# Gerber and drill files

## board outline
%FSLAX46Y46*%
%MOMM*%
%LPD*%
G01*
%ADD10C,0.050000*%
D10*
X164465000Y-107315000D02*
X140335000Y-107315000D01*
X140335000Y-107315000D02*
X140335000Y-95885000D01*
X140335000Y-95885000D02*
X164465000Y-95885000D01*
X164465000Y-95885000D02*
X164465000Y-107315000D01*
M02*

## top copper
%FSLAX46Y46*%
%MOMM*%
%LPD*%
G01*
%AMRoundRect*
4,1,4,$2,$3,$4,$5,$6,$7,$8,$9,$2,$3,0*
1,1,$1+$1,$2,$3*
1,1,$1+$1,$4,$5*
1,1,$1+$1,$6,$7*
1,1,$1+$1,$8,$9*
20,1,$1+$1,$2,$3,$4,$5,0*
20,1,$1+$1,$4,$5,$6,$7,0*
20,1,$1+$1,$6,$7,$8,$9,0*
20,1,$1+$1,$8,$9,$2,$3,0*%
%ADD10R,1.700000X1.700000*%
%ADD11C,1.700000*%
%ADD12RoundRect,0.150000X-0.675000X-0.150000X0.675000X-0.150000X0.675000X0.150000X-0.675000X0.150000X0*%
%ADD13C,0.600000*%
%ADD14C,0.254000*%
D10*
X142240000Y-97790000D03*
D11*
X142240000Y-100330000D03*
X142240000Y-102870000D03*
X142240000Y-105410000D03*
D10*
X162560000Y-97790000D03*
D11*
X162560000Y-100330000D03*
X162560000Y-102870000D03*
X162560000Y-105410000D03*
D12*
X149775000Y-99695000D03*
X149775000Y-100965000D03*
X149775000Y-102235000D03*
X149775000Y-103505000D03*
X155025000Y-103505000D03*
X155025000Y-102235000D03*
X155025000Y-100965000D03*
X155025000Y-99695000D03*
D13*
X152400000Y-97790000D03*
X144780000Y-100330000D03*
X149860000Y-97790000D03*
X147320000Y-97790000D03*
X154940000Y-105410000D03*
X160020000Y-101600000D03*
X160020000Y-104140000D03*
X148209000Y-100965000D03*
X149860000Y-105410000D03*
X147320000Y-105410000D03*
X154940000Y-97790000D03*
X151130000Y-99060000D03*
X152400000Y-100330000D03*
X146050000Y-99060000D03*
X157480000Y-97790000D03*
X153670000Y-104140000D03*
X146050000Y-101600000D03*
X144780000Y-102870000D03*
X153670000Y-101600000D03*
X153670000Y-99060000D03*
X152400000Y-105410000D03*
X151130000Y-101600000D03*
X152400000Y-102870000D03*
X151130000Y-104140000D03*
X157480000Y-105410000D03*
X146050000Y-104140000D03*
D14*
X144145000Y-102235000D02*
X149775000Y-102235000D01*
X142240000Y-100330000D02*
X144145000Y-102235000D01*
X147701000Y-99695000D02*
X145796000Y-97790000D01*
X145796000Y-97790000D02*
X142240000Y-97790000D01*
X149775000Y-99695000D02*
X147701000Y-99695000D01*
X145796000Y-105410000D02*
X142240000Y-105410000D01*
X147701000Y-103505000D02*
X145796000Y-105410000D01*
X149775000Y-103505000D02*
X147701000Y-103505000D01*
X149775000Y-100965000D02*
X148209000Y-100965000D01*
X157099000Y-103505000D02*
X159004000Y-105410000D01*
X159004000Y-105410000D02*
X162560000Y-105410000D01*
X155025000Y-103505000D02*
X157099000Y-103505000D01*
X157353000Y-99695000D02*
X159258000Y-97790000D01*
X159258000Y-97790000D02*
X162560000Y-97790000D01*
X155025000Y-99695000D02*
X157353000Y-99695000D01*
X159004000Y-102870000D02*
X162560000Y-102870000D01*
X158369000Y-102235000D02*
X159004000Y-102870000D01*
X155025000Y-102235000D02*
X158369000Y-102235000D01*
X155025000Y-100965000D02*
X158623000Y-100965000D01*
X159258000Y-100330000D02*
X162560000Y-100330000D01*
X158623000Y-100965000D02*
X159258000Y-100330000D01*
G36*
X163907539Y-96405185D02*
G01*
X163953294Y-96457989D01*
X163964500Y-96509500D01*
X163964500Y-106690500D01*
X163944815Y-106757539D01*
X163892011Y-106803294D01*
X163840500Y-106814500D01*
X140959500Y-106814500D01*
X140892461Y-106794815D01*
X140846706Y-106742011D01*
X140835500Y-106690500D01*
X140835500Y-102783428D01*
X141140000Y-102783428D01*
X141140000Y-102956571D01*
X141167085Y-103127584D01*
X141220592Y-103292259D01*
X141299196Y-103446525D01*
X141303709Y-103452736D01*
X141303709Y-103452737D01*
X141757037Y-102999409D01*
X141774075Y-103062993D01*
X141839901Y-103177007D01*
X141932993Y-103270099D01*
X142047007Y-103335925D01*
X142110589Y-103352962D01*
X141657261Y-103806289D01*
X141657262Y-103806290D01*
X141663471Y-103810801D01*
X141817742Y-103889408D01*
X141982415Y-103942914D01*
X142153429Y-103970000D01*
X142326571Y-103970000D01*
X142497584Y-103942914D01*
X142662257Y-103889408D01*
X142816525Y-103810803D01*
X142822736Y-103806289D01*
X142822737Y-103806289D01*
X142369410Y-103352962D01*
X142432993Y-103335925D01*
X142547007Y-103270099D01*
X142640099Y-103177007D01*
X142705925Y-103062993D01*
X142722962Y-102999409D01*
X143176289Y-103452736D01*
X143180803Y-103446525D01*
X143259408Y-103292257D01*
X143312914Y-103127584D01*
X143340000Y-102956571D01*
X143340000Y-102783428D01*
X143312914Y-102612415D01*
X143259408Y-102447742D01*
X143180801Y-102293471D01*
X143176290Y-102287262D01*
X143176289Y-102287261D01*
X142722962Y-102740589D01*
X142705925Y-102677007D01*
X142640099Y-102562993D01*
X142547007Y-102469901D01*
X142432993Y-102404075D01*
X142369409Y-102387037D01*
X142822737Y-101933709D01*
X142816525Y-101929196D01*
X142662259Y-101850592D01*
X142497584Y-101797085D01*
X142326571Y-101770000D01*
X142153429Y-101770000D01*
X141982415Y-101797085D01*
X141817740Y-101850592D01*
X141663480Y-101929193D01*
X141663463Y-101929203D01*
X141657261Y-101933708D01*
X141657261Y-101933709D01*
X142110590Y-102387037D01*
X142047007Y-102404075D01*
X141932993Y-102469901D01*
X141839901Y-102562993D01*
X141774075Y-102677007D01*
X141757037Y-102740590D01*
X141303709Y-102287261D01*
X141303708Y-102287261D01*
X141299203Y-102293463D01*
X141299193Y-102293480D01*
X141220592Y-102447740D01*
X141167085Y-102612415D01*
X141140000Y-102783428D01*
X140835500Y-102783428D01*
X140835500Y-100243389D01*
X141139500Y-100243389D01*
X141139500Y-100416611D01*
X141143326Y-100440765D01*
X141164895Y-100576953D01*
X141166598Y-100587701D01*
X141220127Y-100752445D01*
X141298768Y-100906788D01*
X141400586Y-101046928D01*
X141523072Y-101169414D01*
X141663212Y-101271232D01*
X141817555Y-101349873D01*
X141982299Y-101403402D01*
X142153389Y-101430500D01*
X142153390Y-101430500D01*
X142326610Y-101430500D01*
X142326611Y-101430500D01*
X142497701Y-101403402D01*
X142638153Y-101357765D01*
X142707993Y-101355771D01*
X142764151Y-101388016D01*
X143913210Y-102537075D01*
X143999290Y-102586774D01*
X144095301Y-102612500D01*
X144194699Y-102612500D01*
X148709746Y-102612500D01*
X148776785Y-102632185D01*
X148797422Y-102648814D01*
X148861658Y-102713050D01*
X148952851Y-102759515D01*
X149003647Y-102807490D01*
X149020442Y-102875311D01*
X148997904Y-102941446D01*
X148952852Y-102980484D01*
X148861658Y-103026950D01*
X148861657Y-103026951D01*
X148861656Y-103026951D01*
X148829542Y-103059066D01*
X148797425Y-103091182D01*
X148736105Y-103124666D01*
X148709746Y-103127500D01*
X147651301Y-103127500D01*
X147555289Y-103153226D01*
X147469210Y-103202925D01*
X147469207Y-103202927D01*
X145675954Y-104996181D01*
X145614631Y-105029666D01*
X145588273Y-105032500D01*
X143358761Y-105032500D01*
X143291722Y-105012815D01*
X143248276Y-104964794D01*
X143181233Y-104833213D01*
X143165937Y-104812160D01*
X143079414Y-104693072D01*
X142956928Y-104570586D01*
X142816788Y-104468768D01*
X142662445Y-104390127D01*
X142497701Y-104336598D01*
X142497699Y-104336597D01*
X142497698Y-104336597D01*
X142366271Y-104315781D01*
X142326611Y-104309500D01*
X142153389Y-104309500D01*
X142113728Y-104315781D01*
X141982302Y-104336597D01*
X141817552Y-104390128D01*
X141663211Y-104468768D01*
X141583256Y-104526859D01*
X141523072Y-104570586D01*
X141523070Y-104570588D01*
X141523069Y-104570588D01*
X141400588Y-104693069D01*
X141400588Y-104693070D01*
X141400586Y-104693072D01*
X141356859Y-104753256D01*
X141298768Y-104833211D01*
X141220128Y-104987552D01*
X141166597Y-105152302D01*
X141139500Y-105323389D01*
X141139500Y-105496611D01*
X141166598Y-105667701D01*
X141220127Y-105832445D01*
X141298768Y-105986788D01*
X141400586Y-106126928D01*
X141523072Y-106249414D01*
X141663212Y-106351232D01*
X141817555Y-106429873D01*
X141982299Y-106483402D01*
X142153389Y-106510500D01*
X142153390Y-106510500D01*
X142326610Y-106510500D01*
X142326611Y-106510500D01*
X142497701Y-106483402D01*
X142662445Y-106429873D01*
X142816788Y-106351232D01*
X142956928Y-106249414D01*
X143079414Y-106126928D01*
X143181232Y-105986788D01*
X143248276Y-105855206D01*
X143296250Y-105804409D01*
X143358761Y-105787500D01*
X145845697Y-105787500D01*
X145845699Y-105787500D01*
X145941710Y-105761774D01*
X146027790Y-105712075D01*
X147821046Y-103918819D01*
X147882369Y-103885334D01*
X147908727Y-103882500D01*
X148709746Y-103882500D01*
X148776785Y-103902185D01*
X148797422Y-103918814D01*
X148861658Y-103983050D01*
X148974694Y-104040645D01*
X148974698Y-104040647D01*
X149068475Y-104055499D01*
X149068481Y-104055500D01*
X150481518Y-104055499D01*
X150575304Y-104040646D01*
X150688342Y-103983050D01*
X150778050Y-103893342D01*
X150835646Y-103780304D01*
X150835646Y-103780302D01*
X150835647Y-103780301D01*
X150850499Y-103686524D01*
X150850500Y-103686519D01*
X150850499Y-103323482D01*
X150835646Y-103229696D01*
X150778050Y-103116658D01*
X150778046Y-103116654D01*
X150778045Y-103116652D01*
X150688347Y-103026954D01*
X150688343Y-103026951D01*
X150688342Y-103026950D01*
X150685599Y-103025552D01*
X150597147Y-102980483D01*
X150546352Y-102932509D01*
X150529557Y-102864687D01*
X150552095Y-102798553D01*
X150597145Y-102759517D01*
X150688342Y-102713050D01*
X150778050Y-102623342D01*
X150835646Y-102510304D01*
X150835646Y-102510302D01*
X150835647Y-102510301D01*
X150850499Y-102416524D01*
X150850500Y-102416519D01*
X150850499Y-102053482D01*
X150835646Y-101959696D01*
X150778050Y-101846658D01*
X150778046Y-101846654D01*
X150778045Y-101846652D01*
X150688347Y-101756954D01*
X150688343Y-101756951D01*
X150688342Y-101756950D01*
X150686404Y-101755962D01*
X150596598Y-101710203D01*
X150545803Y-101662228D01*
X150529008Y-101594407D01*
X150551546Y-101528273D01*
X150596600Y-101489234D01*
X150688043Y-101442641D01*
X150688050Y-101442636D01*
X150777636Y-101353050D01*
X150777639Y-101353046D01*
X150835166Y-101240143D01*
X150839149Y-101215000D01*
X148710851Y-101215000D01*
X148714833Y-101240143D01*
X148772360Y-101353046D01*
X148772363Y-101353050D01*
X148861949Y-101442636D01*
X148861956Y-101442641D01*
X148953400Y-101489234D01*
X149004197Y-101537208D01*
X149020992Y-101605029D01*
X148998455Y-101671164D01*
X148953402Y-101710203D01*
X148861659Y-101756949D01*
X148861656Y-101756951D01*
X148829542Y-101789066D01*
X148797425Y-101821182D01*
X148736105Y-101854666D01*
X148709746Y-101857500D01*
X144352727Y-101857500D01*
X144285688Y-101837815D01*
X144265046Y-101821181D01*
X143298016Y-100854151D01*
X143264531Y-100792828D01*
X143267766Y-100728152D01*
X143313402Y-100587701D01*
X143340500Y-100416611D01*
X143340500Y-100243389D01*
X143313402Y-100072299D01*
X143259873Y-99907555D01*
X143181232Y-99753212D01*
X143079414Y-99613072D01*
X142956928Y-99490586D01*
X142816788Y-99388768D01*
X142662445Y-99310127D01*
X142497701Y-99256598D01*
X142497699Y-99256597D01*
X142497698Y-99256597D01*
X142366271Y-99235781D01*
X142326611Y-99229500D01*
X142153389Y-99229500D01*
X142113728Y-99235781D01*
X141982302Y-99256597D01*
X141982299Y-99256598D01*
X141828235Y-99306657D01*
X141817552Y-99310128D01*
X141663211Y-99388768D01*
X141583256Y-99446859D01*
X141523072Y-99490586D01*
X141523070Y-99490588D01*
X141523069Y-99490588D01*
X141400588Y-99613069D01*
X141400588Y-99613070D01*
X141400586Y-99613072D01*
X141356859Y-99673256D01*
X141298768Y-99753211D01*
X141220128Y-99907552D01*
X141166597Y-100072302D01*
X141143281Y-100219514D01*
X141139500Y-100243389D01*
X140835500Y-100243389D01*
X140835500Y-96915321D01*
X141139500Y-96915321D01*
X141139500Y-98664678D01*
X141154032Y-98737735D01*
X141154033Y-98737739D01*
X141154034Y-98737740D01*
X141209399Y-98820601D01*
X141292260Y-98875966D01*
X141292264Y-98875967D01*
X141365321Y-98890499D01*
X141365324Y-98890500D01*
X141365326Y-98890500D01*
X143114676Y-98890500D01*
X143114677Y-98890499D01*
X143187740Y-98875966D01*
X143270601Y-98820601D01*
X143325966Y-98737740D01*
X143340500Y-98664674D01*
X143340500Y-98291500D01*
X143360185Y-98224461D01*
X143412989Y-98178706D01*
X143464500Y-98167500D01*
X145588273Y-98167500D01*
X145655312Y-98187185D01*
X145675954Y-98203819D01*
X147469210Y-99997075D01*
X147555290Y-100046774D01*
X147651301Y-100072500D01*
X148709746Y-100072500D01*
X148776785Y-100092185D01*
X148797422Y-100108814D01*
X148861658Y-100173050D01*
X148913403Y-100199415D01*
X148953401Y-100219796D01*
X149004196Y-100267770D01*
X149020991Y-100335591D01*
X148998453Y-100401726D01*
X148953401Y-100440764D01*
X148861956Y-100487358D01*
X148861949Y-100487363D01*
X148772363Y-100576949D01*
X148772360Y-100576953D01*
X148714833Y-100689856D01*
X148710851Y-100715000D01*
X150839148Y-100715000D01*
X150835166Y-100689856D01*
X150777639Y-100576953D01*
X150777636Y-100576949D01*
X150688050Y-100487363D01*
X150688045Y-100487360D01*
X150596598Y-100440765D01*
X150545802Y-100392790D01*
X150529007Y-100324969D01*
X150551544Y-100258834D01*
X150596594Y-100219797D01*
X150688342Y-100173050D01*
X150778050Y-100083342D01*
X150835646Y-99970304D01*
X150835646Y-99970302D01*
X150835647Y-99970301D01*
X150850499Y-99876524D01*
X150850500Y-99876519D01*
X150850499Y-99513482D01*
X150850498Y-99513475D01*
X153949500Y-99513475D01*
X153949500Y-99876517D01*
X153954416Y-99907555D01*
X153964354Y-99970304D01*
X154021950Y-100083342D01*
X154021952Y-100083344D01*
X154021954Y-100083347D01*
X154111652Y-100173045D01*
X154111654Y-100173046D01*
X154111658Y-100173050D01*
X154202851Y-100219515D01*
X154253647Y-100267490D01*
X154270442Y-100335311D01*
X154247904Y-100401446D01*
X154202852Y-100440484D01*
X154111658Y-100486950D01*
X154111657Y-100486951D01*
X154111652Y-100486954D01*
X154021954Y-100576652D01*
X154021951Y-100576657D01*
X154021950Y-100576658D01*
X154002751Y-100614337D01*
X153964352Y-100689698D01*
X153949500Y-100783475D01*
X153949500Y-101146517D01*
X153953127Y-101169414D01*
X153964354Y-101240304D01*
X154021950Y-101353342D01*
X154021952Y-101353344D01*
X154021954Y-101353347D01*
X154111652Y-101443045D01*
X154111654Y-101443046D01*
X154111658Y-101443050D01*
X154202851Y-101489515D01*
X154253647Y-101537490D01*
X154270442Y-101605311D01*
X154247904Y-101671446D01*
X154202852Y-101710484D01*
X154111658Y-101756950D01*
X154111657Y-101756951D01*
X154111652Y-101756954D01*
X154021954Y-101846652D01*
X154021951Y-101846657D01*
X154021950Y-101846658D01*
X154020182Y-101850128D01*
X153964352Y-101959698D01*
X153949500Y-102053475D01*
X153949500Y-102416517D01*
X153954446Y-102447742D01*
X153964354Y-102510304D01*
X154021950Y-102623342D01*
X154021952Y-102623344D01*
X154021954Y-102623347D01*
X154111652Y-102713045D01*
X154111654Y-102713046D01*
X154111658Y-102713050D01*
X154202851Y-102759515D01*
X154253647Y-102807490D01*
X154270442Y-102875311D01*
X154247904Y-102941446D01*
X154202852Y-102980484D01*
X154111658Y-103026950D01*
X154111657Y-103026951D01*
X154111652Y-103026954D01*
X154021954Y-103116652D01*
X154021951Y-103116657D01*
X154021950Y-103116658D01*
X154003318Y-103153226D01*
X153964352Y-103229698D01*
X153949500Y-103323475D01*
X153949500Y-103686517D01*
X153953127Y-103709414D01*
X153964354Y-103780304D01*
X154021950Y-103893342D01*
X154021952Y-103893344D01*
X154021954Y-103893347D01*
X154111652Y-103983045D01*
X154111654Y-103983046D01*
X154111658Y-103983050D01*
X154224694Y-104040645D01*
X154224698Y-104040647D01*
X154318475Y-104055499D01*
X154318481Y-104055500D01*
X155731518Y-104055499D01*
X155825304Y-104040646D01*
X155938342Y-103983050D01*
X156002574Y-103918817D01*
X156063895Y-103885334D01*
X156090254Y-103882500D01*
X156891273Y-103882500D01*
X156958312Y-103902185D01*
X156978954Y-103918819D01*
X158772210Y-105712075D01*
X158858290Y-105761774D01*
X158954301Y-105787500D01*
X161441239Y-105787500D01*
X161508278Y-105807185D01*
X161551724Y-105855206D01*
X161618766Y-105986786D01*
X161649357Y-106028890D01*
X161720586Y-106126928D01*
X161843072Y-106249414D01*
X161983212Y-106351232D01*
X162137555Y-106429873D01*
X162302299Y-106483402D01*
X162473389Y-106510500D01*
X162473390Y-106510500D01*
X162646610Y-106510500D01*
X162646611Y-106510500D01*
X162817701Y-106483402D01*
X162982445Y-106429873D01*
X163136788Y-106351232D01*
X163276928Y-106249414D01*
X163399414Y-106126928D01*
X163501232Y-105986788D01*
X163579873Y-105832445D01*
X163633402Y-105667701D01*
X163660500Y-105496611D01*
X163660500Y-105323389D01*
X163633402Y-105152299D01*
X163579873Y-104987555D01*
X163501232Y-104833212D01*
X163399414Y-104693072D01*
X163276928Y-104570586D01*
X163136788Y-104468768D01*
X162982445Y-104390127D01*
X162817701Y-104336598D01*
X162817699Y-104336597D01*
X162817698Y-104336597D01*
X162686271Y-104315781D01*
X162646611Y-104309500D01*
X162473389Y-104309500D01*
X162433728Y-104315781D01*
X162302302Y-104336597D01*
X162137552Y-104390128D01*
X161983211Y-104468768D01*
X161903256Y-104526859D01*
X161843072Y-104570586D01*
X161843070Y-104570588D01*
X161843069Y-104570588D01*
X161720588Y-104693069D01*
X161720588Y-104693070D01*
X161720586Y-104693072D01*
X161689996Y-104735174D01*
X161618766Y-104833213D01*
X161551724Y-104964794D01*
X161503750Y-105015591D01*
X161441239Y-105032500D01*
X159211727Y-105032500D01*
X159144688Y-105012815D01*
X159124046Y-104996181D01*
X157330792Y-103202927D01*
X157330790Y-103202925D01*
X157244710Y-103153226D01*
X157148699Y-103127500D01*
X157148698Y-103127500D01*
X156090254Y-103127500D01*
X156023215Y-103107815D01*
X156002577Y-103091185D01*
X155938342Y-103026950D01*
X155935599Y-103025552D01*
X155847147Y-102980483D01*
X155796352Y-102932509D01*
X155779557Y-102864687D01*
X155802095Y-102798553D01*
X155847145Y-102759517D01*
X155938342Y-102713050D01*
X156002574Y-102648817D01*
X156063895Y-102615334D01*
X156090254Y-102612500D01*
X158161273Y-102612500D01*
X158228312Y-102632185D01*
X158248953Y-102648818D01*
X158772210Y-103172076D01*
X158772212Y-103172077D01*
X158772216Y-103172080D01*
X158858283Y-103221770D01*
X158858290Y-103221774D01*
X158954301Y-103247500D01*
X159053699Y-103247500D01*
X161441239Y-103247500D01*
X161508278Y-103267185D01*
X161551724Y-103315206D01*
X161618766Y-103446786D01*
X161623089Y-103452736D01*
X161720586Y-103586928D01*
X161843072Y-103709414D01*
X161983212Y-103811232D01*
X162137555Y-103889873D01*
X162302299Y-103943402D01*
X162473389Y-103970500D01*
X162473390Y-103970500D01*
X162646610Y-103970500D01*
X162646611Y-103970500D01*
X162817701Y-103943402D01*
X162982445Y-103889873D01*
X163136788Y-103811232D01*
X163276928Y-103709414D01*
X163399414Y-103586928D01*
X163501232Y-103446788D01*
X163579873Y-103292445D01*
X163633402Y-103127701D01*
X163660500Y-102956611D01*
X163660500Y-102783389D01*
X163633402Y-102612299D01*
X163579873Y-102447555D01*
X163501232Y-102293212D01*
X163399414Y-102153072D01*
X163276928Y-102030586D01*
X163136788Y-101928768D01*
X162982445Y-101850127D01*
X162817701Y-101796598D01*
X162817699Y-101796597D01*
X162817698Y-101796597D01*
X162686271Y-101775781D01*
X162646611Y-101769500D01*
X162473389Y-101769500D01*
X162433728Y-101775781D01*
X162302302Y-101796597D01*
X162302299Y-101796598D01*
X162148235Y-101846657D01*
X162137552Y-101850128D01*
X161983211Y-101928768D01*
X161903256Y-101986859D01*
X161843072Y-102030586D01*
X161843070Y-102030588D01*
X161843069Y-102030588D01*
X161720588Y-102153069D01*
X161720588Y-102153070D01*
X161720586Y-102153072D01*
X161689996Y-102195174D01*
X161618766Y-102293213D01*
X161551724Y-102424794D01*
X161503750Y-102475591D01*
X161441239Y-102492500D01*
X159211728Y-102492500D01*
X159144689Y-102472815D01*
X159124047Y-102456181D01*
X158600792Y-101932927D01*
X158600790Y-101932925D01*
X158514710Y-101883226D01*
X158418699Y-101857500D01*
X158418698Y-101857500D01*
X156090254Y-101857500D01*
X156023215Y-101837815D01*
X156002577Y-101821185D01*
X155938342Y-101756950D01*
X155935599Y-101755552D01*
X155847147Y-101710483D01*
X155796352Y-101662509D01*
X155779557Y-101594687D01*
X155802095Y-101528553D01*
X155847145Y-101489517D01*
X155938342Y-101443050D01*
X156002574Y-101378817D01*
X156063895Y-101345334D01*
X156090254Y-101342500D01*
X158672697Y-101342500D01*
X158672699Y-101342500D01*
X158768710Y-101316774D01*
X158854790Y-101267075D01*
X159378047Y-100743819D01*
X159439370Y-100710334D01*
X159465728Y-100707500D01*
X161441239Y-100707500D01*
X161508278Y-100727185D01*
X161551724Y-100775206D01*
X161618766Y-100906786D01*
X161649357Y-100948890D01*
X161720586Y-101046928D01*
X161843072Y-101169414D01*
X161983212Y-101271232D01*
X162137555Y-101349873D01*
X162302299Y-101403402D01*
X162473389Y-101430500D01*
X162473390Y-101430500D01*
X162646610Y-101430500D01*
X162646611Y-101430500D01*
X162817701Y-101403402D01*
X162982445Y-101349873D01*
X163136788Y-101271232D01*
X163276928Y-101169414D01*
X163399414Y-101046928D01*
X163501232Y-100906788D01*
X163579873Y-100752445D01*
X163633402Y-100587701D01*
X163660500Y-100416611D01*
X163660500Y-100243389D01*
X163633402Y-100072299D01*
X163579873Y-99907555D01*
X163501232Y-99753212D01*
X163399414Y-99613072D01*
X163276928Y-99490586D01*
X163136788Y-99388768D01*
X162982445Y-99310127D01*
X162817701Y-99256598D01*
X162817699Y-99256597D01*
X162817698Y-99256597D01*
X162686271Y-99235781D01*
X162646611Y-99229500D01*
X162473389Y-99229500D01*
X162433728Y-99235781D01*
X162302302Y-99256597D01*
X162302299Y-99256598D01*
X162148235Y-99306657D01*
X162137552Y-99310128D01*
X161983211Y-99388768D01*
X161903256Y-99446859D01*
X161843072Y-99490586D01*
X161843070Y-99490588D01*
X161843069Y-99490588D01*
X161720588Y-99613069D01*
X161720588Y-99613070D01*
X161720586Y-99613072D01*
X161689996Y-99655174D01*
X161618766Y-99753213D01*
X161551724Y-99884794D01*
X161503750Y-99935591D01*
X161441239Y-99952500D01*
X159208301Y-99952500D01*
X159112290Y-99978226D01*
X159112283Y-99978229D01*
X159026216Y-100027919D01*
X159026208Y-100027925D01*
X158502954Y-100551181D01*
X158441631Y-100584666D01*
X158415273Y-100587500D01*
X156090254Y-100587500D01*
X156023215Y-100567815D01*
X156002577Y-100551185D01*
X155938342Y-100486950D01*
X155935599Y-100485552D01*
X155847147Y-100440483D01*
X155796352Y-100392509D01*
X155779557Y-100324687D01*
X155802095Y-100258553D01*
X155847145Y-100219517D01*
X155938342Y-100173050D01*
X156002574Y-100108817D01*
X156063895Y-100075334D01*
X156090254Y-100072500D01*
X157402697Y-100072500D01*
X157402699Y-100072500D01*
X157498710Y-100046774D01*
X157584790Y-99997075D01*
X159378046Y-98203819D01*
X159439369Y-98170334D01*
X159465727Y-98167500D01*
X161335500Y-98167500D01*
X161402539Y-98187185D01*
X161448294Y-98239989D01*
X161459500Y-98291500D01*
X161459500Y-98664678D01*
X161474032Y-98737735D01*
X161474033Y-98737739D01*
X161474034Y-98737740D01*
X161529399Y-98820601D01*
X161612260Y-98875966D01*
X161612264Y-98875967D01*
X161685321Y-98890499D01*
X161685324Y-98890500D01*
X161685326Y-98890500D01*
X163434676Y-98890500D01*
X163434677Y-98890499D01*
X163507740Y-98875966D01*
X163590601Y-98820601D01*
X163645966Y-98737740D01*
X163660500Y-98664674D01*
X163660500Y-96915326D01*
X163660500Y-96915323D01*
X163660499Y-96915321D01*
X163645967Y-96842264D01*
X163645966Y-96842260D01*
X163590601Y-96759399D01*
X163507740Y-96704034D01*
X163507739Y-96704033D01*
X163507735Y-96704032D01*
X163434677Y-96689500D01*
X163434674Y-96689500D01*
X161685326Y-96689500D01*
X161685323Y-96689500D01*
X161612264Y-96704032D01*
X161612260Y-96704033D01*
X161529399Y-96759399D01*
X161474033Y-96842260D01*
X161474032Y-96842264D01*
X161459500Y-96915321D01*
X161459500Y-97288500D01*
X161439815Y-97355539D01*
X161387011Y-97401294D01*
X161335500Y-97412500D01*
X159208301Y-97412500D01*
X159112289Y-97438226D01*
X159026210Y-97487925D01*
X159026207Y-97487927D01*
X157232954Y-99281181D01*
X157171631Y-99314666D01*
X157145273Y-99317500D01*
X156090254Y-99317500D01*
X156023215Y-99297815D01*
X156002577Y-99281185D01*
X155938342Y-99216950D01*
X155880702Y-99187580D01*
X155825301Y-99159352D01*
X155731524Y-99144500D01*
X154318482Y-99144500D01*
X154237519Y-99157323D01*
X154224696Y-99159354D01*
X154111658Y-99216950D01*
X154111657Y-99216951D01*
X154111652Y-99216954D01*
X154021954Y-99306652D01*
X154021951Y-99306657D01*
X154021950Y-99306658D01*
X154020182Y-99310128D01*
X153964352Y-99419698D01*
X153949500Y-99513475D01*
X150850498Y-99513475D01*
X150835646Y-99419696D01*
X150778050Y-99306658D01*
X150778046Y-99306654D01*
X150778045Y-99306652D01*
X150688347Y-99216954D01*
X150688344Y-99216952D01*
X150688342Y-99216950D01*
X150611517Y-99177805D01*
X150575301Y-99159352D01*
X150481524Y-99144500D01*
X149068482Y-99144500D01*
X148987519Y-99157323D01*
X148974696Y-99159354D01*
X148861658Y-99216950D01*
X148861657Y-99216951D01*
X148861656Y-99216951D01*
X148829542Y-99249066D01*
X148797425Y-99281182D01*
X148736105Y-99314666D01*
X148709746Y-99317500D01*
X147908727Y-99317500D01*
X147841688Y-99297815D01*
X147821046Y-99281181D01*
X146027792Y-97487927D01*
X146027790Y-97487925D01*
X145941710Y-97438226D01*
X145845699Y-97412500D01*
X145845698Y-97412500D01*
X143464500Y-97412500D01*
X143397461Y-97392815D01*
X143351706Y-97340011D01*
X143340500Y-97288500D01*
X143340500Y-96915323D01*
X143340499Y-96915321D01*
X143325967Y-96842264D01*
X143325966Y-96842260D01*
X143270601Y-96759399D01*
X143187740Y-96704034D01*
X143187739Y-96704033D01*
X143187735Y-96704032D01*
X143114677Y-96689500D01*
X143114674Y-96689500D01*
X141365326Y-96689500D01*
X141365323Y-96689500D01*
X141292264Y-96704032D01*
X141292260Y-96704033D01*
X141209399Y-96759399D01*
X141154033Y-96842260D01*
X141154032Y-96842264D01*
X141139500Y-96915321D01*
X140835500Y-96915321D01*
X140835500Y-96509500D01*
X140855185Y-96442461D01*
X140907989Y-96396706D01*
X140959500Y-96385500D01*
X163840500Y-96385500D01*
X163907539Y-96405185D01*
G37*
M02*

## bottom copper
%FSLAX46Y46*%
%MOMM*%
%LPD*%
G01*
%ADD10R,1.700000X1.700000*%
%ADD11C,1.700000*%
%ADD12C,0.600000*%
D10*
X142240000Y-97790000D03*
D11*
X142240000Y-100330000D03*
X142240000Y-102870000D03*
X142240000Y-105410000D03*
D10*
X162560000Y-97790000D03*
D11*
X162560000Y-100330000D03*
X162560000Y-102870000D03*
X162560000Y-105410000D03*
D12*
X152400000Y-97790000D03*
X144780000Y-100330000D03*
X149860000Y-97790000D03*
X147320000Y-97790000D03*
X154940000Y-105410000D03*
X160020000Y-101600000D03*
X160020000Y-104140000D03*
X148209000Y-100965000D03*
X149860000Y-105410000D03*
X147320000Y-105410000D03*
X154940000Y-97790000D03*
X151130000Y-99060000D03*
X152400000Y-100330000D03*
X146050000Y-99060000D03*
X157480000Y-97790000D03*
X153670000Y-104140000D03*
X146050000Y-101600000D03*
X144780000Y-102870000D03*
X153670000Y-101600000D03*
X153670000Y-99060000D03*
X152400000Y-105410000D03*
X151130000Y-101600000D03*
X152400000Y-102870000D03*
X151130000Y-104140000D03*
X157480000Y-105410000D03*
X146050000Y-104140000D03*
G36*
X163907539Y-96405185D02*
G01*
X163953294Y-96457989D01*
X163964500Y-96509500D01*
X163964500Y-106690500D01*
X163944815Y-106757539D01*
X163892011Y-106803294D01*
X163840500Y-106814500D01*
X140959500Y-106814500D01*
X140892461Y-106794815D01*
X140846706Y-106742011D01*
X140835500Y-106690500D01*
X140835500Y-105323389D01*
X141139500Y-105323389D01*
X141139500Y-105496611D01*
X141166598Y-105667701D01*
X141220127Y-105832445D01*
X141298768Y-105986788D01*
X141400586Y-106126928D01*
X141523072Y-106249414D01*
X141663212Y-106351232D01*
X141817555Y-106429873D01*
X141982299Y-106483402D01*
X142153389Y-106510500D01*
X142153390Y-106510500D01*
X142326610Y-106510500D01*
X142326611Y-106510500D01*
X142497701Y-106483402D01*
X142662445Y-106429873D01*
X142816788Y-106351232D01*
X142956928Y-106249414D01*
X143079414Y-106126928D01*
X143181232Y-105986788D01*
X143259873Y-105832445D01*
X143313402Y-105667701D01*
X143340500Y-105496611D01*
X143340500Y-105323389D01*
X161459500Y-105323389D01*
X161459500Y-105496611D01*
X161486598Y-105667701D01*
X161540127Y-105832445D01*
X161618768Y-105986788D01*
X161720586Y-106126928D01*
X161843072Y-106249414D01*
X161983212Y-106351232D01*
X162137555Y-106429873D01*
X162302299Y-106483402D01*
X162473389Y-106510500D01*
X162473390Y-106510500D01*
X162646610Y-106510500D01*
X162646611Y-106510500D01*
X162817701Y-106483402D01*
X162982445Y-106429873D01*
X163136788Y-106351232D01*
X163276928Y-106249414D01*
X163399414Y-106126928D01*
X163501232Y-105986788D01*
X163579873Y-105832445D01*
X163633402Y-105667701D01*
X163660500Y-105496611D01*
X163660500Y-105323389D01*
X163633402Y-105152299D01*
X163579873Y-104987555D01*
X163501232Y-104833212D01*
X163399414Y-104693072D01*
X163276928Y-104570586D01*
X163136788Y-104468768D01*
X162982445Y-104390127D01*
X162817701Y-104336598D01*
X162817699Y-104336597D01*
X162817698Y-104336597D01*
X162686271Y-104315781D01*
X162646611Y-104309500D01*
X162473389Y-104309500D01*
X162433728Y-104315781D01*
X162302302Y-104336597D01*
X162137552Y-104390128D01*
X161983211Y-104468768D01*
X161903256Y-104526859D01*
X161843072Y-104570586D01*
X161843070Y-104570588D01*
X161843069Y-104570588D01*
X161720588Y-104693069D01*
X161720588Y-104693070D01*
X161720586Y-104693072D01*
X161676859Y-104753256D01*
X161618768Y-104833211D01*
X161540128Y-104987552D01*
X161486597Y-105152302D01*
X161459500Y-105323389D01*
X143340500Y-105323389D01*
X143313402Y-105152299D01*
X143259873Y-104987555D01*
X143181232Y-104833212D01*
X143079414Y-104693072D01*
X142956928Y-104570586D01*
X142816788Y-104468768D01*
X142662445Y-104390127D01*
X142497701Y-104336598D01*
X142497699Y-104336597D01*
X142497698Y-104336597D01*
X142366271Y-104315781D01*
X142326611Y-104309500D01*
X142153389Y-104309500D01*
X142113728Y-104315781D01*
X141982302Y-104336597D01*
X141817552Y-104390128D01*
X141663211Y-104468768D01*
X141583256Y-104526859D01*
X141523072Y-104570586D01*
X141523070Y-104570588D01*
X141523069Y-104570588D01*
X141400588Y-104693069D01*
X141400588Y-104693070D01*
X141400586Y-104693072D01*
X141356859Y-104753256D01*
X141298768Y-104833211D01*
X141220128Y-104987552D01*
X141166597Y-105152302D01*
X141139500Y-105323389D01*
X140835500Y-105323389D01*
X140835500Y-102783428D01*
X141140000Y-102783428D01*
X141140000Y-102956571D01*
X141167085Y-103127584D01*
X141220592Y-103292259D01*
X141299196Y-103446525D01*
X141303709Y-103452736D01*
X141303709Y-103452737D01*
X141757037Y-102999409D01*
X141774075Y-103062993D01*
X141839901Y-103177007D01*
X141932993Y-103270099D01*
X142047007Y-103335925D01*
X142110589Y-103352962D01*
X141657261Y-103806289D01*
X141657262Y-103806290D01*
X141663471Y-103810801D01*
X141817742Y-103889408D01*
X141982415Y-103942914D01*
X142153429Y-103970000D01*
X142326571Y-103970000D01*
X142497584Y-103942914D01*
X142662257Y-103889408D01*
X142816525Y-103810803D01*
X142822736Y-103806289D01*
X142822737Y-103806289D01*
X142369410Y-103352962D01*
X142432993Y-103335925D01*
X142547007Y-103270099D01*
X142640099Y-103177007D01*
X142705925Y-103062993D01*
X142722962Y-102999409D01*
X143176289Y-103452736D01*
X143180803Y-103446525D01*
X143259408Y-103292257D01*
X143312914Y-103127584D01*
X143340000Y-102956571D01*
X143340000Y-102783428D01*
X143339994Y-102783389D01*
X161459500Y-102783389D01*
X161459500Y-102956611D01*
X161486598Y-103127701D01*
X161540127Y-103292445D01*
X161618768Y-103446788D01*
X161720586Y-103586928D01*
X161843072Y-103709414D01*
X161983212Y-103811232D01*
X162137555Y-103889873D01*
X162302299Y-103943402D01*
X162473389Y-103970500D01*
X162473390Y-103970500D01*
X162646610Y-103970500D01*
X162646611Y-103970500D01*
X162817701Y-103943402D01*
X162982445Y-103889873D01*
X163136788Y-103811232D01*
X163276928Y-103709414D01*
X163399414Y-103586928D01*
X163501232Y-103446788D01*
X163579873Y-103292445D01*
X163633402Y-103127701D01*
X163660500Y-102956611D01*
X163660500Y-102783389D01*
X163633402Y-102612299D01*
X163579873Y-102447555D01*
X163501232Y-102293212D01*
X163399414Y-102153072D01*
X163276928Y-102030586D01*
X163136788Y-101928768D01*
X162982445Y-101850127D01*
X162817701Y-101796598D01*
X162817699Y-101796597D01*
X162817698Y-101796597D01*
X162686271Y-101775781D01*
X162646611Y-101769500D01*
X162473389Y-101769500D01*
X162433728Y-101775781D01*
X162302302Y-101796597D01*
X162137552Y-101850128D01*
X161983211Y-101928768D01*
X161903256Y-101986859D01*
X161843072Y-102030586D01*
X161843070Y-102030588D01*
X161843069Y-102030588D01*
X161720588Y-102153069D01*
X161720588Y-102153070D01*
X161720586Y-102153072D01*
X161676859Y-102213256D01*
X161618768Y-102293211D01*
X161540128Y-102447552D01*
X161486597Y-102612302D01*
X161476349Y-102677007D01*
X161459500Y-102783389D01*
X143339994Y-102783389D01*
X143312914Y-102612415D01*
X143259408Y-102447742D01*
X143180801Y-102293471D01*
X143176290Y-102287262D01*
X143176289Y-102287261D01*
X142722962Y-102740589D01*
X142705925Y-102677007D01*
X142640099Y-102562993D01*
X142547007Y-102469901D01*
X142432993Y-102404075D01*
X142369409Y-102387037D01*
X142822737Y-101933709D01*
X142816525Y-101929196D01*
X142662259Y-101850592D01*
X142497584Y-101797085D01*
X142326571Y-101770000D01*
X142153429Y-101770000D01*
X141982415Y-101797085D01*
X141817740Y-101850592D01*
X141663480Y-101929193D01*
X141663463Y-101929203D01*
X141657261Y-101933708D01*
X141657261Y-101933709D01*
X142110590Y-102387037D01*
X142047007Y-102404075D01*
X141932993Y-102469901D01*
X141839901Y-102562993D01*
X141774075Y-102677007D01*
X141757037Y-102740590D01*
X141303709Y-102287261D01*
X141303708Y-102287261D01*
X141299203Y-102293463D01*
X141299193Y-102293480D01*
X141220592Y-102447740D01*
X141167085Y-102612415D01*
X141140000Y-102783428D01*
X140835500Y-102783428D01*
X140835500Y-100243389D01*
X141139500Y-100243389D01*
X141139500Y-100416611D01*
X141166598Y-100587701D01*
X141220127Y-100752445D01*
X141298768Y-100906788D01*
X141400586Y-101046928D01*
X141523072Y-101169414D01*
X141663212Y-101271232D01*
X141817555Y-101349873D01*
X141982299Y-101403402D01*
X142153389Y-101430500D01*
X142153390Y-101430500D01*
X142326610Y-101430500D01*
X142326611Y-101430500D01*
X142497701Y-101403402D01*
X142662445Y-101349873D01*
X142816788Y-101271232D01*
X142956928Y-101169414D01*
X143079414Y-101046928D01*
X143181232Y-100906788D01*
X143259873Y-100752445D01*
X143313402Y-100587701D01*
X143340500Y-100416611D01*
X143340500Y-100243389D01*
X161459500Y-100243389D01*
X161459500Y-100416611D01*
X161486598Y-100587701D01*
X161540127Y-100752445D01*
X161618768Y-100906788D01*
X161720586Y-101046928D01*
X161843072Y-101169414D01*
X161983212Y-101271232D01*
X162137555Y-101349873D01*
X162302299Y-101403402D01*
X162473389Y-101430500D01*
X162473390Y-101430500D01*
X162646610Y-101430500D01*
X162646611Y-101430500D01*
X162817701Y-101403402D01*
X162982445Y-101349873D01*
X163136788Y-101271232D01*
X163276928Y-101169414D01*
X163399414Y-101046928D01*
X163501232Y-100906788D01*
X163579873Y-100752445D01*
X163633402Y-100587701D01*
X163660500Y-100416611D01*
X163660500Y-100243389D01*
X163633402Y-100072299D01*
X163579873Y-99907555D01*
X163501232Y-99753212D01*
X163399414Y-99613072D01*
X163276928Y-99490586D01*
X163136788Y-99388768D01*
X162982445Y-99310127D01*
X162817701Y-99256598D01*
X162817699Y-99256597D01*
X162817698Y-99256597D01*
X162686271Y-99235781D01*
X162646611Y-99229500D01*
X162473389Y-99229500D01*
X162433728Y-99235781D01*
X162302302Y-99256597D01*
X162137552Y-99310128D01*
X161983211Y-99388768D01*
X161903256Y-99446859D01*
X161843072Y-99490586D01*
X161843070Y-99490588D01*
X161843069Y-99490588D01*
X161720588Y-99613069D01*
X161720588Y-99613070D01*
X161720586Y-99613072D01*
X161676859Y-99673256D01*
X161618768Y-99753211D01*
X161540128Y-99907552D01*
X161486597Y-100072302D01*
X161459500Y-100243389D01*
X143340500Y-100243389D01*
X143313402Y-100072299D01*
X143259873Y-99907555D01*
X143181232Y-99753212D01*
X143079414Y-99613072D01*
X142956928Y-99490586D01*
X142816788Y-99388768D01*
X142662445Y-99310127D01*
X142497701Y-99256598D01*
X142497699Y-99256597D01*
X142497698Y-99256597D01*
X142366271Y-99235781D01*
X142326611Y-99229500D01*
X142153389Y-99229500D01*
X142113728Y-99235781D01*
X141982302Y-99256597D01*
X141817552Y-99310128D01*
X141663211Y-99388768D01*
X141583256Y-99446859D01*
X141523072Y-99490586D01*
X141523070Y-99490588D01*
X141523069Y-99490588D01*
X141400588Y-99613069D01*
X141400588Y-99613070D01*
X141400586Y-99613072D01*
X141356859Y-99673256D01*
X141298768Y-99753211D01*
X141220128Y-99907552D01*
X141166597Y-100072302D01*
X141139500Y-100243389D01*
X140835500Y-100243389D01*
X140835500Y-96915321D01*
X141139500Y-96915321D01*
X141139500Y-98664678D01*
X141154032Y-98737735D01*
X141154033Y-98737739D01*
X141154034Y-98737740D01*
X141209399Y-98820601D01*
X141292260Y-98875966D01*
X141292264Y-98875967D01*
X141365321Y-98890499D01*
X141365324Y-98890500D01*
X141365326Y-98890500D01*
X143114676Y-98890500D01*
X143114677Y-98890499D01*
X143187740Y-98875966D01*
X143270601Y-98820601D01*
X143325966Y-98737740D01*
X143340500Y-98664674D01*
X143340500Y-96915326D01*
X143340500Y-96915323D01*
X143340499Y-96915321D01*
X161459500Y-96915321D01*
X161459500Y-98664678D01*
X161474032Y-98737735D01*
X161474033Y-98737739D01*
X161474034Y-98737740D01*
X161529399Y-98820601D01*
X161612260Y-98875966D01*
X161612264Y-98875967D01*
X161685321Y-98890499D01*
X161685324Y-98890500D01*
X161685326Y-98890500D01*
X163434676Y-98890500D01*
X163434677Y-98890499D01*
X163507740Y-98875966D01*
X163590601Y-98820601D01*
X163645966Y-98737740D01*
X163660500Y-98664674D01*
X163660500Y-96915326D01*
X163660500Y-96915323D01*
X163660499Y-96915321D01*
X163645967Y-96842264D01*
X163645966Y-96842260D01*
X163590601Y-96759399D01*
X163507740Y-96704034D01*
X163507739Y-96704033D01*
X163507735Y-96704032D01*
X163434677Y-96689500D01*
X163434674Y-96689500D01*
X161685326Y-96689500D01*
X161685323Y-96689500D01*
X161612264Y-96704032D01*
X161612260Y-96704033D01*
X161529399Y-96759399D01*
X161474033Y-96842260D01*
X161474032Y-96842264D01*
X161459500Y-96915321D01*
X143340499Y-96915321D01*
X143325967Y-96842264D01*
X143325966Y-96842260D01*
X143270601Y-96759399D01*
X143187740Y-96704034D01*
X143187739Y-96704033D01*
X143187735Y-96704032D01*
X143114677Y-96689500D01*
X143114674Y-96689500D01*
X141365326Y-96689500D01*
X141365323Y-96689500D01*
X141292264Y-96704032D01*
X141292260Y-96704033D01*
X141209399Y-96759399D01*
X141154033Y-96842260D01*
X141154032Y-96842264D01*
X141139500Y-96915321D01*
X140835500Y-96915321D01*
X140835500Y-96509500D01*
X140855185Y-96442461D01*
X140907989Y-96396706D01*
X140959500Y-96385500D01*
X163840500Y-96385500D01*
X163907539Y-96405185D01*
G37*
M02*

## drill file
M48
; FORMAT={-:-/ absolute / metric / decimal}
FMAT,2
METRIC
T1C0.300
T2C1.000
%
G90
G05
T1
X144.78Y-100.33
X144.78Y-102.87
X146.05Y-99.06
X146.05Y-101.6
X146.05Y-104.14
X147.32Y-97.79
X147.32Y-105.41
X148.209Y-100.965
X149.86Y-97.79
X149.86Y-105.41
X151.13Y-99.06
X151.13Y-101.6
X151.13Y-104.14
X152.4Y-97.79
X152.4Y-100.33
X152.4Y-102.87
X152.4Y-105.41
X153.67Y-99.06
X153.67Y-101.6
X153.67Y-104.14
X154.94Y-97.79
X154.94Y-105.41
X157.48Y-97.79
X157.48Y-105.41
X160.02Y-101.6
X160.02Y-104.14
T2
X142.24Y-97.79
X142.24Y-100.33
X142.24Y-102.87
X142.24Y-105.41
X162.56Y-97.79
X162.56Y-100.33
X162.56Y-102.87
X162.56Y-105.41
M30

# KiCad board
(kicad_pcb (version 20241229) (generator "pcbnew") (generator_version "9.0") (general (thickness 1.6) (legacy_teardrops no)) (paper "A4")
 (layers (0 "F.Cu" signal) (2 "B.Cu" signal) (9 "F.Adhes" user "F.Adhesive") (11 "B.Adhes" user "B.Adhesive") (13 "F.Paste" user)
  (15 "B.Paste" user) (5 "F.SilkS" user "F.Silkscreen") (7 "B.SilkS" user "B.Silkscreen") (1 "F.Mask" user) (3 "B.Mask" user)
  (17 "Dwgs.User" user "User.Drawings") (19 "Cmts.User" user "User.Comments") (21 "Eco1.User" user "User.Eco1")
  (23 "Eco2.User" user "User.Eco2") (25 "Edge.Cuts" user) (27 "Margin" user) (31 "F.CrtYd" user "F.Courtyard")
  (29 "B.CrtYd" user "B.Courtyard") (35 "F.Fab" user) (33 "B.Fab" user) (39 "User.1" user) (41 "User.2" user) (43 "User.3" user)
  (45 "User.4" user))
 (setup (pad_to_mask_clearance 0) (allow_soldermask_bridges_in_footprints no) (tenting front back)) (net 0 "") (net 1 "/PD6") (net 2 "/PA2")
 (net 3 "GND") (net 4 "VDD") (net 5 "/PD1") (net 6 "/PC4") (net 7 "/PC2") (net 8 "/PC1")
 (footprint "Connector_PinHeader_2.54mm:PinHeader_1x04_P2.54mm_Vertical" (layer "F.Cu") (at 142.24 97.79)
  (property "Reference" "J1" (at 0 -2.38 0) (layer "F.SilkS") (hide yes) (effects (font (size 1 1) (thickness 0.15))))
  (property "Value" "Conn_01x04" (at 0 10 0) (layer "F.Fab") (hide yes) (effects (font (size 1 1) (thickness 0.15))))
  (pad "1" thru_hole rect (at 0 0) (size 1.7 1.7) (drill 1) (layers "*.Cu" "*.Mask") (remove_unused_layers no) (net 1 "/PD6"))
  (pad "2" thru_hole circle (at 0 2.54) (size 1.7 1.7) (drill 1) (layers "*.Cu" "*.Mask") (remove_unused_layers no) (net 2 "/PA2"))
  (pad "3" thru_hole circle (at 0 5.08) (size 1.7 1.7) (drill 1) (layers "*.Cu" "*.Mask") (remove_unused_layers no) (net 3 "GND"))
  (pad "4" thru_hole circle (at 0 7.62) (size 1.7 1.7) (drill 1) (layers "*.Cu" "*.Mask") (remove_unused_layers no) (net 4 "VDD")))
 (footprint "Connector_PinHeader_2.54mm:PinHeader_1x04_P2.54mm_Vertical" (layer "F.Cu") (at 162.56 97.79)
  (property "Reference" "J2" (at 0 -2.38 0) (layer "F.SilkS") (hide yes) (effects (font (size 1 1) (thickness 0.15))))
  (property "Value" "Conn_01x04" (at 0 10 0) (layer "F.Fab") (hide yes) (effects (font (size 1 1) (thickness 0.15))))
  (pad "1" thru_hole rect (at 0 0) (size 1.7 1.7) (drill 1) (layers "*.Cu" "*.Mask") (remove_unused_layers no) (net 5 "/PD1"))
  (pad "2" thru_hole circle (at 0 2.54) (size 1.7 1.7) (drill 1) (layers "*.Cu" "*.Mask") (remove_unused_layers no) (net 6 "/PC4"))
  (pad "3" thru_hole circle (at 0 5.08) (size 1.7 1.7) (drill 1) (layers "*.Cu" "*.Mask") (remove_unused_layers no) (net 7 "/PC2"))
  (pad "4" thru_hole circle (at 0 7.62) (size 1.7 1.7) (drill 1) (layers "*.Cu" "*.Mask") (remove_unused_layers no) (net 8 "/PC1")))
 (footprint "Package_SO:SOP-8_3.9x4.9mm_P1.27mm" (layer "F.Cu") (at 152.4 101.6)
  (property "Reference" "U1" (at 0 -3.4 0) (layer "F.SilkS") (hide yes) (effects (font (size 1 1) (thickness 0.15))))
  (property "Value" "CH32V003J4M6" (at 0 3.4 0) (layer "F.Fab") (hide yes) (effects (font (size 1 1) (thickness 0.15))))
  (pad "1" smd roundrect (at -2.625 -1.905) (size 1.65 0.6) (layers "F.Cu" "F.Mask" "F.Paste") (roundrect_rratio 0.25) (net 1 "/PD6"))
  (pad "2" smd roundrect (at -2.625 -0.635) (size 1.65 0.6) (layers "F.Cu" "F.Mask" "F.Paste") (roundrect_rratio 0.25) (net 3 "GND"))
  (pad "3" smd roundrect (at -2.625 0.635) (size 1.65 0.6) (layers "F.Cu" "F.Mask" "F.Paste") (roundrect_rratio 0.25) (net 2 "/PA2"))
  (pad "4" smd roundrect (at -2.625 1.905) (size 1.65 0.6) (layers "F.Cu" "F.Mask" "F.Paste") (roundrect_rratio 0.25) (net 4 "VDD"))
  (pad "5" smd roundrect (at 2.625 1.905) (size 1.65 0.6) (layers "F.Cu" "F.Mask" "F.Paste") (roundrect_rratio 0.25) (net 8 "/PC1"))
  (pad "6" smd roundrect (at 2.625 0.635) (size 1.65 0.6) (layers "F.Cu" "F.Mask" "F.Paste") (roundrect_rratio 0.25) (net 7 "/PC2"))
  (pad "7" smd roundrect (at 2.625 -0.635) (size 1.65 0.6) (layers "F.Cu" "F.Mask" "F.Paste") (roundrect_rratio 0.25) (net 6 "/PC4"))
  (pad "8" smd roundrect (at 2.625 -1.905) (size 1.65 0.6) (layers "F.Cu" "F.Mask" "F.Paste") (roundrect_rratio 0.25) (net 5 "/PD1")))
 (gr_line (start 164.465 107.315) (end 140.335 107.315) (stroke (width 0.05) (type default)) (layer "Edge.Cuts"))
 (gr_line (start 140.335 107.315) (end 140.335 95.885) (stroke (width 0.05) (type default)) (layer "Edge.Cuts"))
 (gr_line (start 140.335 95.885) (end 164.465 95.885) (stroke (width 0.05) (type default)) (layer "Edge.Cuts"))
 (gr_line (start 164.465 95.885) (end 164.465 107.315) (stroke (width 0.05) (type default)) (layer "Edge.Cuts"))
 (segment (start 144.145 102.235) (end 149.775 102.235) (width 0.254) (layer "F.Cu") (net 2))
 (segment (start 142.24 100.33) (end 144.145 102.235) (width 0.254) (layer "F.Cu") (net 2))
 (segment (start 147.701 99.695) (end 145.796 97.79) (width 0.254) (layer "F.Cu") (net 1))
 (segment (start 145.796 97.79) (end 142.24 97.79) (width 0.254) (layer "F.Cu") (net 1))
 (segment (start 149.775 99.695) (end 147.701 99.695) (width 0.254) (layer "F.Cu") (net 1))
 (segment (start 145.796 105.41) (end 142.24 105.41) (width 0.254) (layer "F.Cu") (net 4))
 (segment (start 147.701 103.505) (end 145.796 105.41) (width 0.254) (layer "F.Cu") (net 4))
 (segment (start 149.775 103.505) (end 147.701 103.505) (width 0.254) (layer "F.Cu") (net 4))
 (segment (start 149.775 100.965) (end 148.209 100.965) (width 0.254) (layer "F.Cu") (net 3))
 (via (at 152.4 97.79) (size 0.6) (drill 0.3) (layers "F.Cu" "B.Cu") (free yes) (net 3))
 (via (at 144.78 100.33) (size 0.6) (drill 0.3) (layers "F.Cu" "B.Cu") (free yes) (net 3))
 (via (at 149.86 97.79) (size 0.6) (drill 0.3) (layers "F.Cu" "B.Cu") (free yes) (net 3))
 (via (at 147.32 97.79) (size 0.6) (drill 0.3) (layers "F.Cu" "B.Cu") (free yes) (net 3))
 (via (at 154.94 105.41) (size 0.6) (drill 0.3) (layers "F.Cu" "B.Cu") (free yes) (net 3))
 (via (at 160.02 101.6) (size 0.6) (drill 0.3) (layers "F.Cu" "B.Cu") (free yes) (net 3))
 (via (at 160.02 104.14) (size 0.6) (drill 0.3) (layers "F.Cu" "B.Cu") (free yes) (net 3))
 (via (at 148.209 100.965) (size 0.6) (drill 0.3) (layers "F.Cu" "B.Cu") (free yes) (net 3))
 (via (at 149.86 105.41) (size 0.6) (drill 0.3) (layers "F.Cu" "B.Cu") (free yes) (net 3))
 (via (at 147.32 105.41) (size 0.6) (drill 0.3) (layers "F.Cu" "B.Cu") (free yes) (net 3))
 (via (at 154.94 97.79) (size 0.6) (drill 0.3) (layers "F.Cu" "B.Cu") (free yes) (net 3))
 (via (at 151.13 99.06) (size 0.6) (drill 0.3) (layers "F.Cu" "B.Cu") (free yes) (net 3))
 (via (at 152.4 100.33) (size 0.6) (drill 0.3) (layers "F.Cu" "B.Cu") (free yes) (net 3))
 (via (at 146.05 99.06) (size 0.6) (drill 0.3) (layers "F.Cu" "B.Cu") (free yes) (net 3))
 (via (at 157.48 97.79) (size 0.6) (drill 0.3) (layers "F.Cu" "B.Cu") (free yes) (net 3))
 (via (at 153.67 104.14) (size 0.6) (drill 0.3) (layers "F.Cu" "B.Cu") (free yes) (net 3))
 (via (at 146.05 101.6) (size 0.6) (drill 0.3) (layers "F.Cu" "B.Cu") (free yes) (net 3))
 (via (at 144.78 102.87) (size 0.6) (drill 0.3) (layers "F.Cu" "B.Cu") (free yes) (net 3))
 (via (at 153.67 101.6) (size 0.6) (drill 0.3) (layers "F.Cu" "B.Cu") (free yes) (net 3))
 (via (at 153.67 99.06) (size 0.6) (drill 0.3) (layers "F.Cu" "B.Cu") (free yes) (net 3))
 (via (at 152.4 105.41) (size 0.6) (drill 0.3) (layers "F.Cu" "B.Cu") (free yes) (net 3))
 (via (at 151.13 101.6) (size 0.6) (drill 0.3) (layers "F.Cu" "B.Cu") (free yes) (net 3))
 (via (at 152.4 102.87) (size 0.6) (drill 0.3) (layers "F.Cu" "B.Cu") (free yes) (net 3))
 (via (at 151.13 104.14) (size 0.6) (drill 0.3) (layers "F.Cu" "B.Cu") (free yes) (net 3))
 (via (at 157.48 105.41) (size 0.6) (drill 0.3) (layers "F.Cu" "B.Cu") (free yes) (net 3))
 (via (at 146.05 104.14) (size 0.6) (drill 0.3) (layers "F.Cu" "B.Cu") (free yes) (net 3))
 (segment (start 157.099 103.505) (end 159.004 105.41) (width 0.254) (layer "F.Cu") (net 8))
 (segment (start 159.004 105.41) (end 162.56 105.41) (width 0.254) (layer "F.Cu") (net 8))
 (segment (start 155.025 103.505) (end 157.099 103.505) (width 0.254) (layer "F.Cu") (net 8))
 (segment (start 157.353 99.695) (end 159.258 97.79) (width 0.254) (layer "F.Cu") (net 5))
 (segment (start 159.258 97.79) (end 162.56 97.79) (width 0.254) (layer "F.Cu") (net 5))
 (segment (start 155.025 99.695) (end 157.353 99.695) (width 0.254) (layer "F.Cu") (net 5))
 (segment (start 159.004 102.87) (end 162.56 102.87) (width 0.254) (layer "F.Cu") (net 7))
 (segment (start 158.369 102.235) (end 159.004 102.87) (width 0.254) (layer "F.Cu") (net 7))
 (segment (start 155.025 102.235) (end 158.369 102.235) (width 0.254) (layer "F.Cu") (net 7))
 (segment (start 155.025 100.965) (end 158.623 100.965) (width 0.254) (layer "F.Cu") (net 6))
 (segment (start 159.258 100.33) (end 162.56 100.33) (width 0.254) (layer "F.Cu") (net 6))
 (segment (start 158.623 100.965) (end 159.258 100.33) (width 0.254) (layer "F.Cu") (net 6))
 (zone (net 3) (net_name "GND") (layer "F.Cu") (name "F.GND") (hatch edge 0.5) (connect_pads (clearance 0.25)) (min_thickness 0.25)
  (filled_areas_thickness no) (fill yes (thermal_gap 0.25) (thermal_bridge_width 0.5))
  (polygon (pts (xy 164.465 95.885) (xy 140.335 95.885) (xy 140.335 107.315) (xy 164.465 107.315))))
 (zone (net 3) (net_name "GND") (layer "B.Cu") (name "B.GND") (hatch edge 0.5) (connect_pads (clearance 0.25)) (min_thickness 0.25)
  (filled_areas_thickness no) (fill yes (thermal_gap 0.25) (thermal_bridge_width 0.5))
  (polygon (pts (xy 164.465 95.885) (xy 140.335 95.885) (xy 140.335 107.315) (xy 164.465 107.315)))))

